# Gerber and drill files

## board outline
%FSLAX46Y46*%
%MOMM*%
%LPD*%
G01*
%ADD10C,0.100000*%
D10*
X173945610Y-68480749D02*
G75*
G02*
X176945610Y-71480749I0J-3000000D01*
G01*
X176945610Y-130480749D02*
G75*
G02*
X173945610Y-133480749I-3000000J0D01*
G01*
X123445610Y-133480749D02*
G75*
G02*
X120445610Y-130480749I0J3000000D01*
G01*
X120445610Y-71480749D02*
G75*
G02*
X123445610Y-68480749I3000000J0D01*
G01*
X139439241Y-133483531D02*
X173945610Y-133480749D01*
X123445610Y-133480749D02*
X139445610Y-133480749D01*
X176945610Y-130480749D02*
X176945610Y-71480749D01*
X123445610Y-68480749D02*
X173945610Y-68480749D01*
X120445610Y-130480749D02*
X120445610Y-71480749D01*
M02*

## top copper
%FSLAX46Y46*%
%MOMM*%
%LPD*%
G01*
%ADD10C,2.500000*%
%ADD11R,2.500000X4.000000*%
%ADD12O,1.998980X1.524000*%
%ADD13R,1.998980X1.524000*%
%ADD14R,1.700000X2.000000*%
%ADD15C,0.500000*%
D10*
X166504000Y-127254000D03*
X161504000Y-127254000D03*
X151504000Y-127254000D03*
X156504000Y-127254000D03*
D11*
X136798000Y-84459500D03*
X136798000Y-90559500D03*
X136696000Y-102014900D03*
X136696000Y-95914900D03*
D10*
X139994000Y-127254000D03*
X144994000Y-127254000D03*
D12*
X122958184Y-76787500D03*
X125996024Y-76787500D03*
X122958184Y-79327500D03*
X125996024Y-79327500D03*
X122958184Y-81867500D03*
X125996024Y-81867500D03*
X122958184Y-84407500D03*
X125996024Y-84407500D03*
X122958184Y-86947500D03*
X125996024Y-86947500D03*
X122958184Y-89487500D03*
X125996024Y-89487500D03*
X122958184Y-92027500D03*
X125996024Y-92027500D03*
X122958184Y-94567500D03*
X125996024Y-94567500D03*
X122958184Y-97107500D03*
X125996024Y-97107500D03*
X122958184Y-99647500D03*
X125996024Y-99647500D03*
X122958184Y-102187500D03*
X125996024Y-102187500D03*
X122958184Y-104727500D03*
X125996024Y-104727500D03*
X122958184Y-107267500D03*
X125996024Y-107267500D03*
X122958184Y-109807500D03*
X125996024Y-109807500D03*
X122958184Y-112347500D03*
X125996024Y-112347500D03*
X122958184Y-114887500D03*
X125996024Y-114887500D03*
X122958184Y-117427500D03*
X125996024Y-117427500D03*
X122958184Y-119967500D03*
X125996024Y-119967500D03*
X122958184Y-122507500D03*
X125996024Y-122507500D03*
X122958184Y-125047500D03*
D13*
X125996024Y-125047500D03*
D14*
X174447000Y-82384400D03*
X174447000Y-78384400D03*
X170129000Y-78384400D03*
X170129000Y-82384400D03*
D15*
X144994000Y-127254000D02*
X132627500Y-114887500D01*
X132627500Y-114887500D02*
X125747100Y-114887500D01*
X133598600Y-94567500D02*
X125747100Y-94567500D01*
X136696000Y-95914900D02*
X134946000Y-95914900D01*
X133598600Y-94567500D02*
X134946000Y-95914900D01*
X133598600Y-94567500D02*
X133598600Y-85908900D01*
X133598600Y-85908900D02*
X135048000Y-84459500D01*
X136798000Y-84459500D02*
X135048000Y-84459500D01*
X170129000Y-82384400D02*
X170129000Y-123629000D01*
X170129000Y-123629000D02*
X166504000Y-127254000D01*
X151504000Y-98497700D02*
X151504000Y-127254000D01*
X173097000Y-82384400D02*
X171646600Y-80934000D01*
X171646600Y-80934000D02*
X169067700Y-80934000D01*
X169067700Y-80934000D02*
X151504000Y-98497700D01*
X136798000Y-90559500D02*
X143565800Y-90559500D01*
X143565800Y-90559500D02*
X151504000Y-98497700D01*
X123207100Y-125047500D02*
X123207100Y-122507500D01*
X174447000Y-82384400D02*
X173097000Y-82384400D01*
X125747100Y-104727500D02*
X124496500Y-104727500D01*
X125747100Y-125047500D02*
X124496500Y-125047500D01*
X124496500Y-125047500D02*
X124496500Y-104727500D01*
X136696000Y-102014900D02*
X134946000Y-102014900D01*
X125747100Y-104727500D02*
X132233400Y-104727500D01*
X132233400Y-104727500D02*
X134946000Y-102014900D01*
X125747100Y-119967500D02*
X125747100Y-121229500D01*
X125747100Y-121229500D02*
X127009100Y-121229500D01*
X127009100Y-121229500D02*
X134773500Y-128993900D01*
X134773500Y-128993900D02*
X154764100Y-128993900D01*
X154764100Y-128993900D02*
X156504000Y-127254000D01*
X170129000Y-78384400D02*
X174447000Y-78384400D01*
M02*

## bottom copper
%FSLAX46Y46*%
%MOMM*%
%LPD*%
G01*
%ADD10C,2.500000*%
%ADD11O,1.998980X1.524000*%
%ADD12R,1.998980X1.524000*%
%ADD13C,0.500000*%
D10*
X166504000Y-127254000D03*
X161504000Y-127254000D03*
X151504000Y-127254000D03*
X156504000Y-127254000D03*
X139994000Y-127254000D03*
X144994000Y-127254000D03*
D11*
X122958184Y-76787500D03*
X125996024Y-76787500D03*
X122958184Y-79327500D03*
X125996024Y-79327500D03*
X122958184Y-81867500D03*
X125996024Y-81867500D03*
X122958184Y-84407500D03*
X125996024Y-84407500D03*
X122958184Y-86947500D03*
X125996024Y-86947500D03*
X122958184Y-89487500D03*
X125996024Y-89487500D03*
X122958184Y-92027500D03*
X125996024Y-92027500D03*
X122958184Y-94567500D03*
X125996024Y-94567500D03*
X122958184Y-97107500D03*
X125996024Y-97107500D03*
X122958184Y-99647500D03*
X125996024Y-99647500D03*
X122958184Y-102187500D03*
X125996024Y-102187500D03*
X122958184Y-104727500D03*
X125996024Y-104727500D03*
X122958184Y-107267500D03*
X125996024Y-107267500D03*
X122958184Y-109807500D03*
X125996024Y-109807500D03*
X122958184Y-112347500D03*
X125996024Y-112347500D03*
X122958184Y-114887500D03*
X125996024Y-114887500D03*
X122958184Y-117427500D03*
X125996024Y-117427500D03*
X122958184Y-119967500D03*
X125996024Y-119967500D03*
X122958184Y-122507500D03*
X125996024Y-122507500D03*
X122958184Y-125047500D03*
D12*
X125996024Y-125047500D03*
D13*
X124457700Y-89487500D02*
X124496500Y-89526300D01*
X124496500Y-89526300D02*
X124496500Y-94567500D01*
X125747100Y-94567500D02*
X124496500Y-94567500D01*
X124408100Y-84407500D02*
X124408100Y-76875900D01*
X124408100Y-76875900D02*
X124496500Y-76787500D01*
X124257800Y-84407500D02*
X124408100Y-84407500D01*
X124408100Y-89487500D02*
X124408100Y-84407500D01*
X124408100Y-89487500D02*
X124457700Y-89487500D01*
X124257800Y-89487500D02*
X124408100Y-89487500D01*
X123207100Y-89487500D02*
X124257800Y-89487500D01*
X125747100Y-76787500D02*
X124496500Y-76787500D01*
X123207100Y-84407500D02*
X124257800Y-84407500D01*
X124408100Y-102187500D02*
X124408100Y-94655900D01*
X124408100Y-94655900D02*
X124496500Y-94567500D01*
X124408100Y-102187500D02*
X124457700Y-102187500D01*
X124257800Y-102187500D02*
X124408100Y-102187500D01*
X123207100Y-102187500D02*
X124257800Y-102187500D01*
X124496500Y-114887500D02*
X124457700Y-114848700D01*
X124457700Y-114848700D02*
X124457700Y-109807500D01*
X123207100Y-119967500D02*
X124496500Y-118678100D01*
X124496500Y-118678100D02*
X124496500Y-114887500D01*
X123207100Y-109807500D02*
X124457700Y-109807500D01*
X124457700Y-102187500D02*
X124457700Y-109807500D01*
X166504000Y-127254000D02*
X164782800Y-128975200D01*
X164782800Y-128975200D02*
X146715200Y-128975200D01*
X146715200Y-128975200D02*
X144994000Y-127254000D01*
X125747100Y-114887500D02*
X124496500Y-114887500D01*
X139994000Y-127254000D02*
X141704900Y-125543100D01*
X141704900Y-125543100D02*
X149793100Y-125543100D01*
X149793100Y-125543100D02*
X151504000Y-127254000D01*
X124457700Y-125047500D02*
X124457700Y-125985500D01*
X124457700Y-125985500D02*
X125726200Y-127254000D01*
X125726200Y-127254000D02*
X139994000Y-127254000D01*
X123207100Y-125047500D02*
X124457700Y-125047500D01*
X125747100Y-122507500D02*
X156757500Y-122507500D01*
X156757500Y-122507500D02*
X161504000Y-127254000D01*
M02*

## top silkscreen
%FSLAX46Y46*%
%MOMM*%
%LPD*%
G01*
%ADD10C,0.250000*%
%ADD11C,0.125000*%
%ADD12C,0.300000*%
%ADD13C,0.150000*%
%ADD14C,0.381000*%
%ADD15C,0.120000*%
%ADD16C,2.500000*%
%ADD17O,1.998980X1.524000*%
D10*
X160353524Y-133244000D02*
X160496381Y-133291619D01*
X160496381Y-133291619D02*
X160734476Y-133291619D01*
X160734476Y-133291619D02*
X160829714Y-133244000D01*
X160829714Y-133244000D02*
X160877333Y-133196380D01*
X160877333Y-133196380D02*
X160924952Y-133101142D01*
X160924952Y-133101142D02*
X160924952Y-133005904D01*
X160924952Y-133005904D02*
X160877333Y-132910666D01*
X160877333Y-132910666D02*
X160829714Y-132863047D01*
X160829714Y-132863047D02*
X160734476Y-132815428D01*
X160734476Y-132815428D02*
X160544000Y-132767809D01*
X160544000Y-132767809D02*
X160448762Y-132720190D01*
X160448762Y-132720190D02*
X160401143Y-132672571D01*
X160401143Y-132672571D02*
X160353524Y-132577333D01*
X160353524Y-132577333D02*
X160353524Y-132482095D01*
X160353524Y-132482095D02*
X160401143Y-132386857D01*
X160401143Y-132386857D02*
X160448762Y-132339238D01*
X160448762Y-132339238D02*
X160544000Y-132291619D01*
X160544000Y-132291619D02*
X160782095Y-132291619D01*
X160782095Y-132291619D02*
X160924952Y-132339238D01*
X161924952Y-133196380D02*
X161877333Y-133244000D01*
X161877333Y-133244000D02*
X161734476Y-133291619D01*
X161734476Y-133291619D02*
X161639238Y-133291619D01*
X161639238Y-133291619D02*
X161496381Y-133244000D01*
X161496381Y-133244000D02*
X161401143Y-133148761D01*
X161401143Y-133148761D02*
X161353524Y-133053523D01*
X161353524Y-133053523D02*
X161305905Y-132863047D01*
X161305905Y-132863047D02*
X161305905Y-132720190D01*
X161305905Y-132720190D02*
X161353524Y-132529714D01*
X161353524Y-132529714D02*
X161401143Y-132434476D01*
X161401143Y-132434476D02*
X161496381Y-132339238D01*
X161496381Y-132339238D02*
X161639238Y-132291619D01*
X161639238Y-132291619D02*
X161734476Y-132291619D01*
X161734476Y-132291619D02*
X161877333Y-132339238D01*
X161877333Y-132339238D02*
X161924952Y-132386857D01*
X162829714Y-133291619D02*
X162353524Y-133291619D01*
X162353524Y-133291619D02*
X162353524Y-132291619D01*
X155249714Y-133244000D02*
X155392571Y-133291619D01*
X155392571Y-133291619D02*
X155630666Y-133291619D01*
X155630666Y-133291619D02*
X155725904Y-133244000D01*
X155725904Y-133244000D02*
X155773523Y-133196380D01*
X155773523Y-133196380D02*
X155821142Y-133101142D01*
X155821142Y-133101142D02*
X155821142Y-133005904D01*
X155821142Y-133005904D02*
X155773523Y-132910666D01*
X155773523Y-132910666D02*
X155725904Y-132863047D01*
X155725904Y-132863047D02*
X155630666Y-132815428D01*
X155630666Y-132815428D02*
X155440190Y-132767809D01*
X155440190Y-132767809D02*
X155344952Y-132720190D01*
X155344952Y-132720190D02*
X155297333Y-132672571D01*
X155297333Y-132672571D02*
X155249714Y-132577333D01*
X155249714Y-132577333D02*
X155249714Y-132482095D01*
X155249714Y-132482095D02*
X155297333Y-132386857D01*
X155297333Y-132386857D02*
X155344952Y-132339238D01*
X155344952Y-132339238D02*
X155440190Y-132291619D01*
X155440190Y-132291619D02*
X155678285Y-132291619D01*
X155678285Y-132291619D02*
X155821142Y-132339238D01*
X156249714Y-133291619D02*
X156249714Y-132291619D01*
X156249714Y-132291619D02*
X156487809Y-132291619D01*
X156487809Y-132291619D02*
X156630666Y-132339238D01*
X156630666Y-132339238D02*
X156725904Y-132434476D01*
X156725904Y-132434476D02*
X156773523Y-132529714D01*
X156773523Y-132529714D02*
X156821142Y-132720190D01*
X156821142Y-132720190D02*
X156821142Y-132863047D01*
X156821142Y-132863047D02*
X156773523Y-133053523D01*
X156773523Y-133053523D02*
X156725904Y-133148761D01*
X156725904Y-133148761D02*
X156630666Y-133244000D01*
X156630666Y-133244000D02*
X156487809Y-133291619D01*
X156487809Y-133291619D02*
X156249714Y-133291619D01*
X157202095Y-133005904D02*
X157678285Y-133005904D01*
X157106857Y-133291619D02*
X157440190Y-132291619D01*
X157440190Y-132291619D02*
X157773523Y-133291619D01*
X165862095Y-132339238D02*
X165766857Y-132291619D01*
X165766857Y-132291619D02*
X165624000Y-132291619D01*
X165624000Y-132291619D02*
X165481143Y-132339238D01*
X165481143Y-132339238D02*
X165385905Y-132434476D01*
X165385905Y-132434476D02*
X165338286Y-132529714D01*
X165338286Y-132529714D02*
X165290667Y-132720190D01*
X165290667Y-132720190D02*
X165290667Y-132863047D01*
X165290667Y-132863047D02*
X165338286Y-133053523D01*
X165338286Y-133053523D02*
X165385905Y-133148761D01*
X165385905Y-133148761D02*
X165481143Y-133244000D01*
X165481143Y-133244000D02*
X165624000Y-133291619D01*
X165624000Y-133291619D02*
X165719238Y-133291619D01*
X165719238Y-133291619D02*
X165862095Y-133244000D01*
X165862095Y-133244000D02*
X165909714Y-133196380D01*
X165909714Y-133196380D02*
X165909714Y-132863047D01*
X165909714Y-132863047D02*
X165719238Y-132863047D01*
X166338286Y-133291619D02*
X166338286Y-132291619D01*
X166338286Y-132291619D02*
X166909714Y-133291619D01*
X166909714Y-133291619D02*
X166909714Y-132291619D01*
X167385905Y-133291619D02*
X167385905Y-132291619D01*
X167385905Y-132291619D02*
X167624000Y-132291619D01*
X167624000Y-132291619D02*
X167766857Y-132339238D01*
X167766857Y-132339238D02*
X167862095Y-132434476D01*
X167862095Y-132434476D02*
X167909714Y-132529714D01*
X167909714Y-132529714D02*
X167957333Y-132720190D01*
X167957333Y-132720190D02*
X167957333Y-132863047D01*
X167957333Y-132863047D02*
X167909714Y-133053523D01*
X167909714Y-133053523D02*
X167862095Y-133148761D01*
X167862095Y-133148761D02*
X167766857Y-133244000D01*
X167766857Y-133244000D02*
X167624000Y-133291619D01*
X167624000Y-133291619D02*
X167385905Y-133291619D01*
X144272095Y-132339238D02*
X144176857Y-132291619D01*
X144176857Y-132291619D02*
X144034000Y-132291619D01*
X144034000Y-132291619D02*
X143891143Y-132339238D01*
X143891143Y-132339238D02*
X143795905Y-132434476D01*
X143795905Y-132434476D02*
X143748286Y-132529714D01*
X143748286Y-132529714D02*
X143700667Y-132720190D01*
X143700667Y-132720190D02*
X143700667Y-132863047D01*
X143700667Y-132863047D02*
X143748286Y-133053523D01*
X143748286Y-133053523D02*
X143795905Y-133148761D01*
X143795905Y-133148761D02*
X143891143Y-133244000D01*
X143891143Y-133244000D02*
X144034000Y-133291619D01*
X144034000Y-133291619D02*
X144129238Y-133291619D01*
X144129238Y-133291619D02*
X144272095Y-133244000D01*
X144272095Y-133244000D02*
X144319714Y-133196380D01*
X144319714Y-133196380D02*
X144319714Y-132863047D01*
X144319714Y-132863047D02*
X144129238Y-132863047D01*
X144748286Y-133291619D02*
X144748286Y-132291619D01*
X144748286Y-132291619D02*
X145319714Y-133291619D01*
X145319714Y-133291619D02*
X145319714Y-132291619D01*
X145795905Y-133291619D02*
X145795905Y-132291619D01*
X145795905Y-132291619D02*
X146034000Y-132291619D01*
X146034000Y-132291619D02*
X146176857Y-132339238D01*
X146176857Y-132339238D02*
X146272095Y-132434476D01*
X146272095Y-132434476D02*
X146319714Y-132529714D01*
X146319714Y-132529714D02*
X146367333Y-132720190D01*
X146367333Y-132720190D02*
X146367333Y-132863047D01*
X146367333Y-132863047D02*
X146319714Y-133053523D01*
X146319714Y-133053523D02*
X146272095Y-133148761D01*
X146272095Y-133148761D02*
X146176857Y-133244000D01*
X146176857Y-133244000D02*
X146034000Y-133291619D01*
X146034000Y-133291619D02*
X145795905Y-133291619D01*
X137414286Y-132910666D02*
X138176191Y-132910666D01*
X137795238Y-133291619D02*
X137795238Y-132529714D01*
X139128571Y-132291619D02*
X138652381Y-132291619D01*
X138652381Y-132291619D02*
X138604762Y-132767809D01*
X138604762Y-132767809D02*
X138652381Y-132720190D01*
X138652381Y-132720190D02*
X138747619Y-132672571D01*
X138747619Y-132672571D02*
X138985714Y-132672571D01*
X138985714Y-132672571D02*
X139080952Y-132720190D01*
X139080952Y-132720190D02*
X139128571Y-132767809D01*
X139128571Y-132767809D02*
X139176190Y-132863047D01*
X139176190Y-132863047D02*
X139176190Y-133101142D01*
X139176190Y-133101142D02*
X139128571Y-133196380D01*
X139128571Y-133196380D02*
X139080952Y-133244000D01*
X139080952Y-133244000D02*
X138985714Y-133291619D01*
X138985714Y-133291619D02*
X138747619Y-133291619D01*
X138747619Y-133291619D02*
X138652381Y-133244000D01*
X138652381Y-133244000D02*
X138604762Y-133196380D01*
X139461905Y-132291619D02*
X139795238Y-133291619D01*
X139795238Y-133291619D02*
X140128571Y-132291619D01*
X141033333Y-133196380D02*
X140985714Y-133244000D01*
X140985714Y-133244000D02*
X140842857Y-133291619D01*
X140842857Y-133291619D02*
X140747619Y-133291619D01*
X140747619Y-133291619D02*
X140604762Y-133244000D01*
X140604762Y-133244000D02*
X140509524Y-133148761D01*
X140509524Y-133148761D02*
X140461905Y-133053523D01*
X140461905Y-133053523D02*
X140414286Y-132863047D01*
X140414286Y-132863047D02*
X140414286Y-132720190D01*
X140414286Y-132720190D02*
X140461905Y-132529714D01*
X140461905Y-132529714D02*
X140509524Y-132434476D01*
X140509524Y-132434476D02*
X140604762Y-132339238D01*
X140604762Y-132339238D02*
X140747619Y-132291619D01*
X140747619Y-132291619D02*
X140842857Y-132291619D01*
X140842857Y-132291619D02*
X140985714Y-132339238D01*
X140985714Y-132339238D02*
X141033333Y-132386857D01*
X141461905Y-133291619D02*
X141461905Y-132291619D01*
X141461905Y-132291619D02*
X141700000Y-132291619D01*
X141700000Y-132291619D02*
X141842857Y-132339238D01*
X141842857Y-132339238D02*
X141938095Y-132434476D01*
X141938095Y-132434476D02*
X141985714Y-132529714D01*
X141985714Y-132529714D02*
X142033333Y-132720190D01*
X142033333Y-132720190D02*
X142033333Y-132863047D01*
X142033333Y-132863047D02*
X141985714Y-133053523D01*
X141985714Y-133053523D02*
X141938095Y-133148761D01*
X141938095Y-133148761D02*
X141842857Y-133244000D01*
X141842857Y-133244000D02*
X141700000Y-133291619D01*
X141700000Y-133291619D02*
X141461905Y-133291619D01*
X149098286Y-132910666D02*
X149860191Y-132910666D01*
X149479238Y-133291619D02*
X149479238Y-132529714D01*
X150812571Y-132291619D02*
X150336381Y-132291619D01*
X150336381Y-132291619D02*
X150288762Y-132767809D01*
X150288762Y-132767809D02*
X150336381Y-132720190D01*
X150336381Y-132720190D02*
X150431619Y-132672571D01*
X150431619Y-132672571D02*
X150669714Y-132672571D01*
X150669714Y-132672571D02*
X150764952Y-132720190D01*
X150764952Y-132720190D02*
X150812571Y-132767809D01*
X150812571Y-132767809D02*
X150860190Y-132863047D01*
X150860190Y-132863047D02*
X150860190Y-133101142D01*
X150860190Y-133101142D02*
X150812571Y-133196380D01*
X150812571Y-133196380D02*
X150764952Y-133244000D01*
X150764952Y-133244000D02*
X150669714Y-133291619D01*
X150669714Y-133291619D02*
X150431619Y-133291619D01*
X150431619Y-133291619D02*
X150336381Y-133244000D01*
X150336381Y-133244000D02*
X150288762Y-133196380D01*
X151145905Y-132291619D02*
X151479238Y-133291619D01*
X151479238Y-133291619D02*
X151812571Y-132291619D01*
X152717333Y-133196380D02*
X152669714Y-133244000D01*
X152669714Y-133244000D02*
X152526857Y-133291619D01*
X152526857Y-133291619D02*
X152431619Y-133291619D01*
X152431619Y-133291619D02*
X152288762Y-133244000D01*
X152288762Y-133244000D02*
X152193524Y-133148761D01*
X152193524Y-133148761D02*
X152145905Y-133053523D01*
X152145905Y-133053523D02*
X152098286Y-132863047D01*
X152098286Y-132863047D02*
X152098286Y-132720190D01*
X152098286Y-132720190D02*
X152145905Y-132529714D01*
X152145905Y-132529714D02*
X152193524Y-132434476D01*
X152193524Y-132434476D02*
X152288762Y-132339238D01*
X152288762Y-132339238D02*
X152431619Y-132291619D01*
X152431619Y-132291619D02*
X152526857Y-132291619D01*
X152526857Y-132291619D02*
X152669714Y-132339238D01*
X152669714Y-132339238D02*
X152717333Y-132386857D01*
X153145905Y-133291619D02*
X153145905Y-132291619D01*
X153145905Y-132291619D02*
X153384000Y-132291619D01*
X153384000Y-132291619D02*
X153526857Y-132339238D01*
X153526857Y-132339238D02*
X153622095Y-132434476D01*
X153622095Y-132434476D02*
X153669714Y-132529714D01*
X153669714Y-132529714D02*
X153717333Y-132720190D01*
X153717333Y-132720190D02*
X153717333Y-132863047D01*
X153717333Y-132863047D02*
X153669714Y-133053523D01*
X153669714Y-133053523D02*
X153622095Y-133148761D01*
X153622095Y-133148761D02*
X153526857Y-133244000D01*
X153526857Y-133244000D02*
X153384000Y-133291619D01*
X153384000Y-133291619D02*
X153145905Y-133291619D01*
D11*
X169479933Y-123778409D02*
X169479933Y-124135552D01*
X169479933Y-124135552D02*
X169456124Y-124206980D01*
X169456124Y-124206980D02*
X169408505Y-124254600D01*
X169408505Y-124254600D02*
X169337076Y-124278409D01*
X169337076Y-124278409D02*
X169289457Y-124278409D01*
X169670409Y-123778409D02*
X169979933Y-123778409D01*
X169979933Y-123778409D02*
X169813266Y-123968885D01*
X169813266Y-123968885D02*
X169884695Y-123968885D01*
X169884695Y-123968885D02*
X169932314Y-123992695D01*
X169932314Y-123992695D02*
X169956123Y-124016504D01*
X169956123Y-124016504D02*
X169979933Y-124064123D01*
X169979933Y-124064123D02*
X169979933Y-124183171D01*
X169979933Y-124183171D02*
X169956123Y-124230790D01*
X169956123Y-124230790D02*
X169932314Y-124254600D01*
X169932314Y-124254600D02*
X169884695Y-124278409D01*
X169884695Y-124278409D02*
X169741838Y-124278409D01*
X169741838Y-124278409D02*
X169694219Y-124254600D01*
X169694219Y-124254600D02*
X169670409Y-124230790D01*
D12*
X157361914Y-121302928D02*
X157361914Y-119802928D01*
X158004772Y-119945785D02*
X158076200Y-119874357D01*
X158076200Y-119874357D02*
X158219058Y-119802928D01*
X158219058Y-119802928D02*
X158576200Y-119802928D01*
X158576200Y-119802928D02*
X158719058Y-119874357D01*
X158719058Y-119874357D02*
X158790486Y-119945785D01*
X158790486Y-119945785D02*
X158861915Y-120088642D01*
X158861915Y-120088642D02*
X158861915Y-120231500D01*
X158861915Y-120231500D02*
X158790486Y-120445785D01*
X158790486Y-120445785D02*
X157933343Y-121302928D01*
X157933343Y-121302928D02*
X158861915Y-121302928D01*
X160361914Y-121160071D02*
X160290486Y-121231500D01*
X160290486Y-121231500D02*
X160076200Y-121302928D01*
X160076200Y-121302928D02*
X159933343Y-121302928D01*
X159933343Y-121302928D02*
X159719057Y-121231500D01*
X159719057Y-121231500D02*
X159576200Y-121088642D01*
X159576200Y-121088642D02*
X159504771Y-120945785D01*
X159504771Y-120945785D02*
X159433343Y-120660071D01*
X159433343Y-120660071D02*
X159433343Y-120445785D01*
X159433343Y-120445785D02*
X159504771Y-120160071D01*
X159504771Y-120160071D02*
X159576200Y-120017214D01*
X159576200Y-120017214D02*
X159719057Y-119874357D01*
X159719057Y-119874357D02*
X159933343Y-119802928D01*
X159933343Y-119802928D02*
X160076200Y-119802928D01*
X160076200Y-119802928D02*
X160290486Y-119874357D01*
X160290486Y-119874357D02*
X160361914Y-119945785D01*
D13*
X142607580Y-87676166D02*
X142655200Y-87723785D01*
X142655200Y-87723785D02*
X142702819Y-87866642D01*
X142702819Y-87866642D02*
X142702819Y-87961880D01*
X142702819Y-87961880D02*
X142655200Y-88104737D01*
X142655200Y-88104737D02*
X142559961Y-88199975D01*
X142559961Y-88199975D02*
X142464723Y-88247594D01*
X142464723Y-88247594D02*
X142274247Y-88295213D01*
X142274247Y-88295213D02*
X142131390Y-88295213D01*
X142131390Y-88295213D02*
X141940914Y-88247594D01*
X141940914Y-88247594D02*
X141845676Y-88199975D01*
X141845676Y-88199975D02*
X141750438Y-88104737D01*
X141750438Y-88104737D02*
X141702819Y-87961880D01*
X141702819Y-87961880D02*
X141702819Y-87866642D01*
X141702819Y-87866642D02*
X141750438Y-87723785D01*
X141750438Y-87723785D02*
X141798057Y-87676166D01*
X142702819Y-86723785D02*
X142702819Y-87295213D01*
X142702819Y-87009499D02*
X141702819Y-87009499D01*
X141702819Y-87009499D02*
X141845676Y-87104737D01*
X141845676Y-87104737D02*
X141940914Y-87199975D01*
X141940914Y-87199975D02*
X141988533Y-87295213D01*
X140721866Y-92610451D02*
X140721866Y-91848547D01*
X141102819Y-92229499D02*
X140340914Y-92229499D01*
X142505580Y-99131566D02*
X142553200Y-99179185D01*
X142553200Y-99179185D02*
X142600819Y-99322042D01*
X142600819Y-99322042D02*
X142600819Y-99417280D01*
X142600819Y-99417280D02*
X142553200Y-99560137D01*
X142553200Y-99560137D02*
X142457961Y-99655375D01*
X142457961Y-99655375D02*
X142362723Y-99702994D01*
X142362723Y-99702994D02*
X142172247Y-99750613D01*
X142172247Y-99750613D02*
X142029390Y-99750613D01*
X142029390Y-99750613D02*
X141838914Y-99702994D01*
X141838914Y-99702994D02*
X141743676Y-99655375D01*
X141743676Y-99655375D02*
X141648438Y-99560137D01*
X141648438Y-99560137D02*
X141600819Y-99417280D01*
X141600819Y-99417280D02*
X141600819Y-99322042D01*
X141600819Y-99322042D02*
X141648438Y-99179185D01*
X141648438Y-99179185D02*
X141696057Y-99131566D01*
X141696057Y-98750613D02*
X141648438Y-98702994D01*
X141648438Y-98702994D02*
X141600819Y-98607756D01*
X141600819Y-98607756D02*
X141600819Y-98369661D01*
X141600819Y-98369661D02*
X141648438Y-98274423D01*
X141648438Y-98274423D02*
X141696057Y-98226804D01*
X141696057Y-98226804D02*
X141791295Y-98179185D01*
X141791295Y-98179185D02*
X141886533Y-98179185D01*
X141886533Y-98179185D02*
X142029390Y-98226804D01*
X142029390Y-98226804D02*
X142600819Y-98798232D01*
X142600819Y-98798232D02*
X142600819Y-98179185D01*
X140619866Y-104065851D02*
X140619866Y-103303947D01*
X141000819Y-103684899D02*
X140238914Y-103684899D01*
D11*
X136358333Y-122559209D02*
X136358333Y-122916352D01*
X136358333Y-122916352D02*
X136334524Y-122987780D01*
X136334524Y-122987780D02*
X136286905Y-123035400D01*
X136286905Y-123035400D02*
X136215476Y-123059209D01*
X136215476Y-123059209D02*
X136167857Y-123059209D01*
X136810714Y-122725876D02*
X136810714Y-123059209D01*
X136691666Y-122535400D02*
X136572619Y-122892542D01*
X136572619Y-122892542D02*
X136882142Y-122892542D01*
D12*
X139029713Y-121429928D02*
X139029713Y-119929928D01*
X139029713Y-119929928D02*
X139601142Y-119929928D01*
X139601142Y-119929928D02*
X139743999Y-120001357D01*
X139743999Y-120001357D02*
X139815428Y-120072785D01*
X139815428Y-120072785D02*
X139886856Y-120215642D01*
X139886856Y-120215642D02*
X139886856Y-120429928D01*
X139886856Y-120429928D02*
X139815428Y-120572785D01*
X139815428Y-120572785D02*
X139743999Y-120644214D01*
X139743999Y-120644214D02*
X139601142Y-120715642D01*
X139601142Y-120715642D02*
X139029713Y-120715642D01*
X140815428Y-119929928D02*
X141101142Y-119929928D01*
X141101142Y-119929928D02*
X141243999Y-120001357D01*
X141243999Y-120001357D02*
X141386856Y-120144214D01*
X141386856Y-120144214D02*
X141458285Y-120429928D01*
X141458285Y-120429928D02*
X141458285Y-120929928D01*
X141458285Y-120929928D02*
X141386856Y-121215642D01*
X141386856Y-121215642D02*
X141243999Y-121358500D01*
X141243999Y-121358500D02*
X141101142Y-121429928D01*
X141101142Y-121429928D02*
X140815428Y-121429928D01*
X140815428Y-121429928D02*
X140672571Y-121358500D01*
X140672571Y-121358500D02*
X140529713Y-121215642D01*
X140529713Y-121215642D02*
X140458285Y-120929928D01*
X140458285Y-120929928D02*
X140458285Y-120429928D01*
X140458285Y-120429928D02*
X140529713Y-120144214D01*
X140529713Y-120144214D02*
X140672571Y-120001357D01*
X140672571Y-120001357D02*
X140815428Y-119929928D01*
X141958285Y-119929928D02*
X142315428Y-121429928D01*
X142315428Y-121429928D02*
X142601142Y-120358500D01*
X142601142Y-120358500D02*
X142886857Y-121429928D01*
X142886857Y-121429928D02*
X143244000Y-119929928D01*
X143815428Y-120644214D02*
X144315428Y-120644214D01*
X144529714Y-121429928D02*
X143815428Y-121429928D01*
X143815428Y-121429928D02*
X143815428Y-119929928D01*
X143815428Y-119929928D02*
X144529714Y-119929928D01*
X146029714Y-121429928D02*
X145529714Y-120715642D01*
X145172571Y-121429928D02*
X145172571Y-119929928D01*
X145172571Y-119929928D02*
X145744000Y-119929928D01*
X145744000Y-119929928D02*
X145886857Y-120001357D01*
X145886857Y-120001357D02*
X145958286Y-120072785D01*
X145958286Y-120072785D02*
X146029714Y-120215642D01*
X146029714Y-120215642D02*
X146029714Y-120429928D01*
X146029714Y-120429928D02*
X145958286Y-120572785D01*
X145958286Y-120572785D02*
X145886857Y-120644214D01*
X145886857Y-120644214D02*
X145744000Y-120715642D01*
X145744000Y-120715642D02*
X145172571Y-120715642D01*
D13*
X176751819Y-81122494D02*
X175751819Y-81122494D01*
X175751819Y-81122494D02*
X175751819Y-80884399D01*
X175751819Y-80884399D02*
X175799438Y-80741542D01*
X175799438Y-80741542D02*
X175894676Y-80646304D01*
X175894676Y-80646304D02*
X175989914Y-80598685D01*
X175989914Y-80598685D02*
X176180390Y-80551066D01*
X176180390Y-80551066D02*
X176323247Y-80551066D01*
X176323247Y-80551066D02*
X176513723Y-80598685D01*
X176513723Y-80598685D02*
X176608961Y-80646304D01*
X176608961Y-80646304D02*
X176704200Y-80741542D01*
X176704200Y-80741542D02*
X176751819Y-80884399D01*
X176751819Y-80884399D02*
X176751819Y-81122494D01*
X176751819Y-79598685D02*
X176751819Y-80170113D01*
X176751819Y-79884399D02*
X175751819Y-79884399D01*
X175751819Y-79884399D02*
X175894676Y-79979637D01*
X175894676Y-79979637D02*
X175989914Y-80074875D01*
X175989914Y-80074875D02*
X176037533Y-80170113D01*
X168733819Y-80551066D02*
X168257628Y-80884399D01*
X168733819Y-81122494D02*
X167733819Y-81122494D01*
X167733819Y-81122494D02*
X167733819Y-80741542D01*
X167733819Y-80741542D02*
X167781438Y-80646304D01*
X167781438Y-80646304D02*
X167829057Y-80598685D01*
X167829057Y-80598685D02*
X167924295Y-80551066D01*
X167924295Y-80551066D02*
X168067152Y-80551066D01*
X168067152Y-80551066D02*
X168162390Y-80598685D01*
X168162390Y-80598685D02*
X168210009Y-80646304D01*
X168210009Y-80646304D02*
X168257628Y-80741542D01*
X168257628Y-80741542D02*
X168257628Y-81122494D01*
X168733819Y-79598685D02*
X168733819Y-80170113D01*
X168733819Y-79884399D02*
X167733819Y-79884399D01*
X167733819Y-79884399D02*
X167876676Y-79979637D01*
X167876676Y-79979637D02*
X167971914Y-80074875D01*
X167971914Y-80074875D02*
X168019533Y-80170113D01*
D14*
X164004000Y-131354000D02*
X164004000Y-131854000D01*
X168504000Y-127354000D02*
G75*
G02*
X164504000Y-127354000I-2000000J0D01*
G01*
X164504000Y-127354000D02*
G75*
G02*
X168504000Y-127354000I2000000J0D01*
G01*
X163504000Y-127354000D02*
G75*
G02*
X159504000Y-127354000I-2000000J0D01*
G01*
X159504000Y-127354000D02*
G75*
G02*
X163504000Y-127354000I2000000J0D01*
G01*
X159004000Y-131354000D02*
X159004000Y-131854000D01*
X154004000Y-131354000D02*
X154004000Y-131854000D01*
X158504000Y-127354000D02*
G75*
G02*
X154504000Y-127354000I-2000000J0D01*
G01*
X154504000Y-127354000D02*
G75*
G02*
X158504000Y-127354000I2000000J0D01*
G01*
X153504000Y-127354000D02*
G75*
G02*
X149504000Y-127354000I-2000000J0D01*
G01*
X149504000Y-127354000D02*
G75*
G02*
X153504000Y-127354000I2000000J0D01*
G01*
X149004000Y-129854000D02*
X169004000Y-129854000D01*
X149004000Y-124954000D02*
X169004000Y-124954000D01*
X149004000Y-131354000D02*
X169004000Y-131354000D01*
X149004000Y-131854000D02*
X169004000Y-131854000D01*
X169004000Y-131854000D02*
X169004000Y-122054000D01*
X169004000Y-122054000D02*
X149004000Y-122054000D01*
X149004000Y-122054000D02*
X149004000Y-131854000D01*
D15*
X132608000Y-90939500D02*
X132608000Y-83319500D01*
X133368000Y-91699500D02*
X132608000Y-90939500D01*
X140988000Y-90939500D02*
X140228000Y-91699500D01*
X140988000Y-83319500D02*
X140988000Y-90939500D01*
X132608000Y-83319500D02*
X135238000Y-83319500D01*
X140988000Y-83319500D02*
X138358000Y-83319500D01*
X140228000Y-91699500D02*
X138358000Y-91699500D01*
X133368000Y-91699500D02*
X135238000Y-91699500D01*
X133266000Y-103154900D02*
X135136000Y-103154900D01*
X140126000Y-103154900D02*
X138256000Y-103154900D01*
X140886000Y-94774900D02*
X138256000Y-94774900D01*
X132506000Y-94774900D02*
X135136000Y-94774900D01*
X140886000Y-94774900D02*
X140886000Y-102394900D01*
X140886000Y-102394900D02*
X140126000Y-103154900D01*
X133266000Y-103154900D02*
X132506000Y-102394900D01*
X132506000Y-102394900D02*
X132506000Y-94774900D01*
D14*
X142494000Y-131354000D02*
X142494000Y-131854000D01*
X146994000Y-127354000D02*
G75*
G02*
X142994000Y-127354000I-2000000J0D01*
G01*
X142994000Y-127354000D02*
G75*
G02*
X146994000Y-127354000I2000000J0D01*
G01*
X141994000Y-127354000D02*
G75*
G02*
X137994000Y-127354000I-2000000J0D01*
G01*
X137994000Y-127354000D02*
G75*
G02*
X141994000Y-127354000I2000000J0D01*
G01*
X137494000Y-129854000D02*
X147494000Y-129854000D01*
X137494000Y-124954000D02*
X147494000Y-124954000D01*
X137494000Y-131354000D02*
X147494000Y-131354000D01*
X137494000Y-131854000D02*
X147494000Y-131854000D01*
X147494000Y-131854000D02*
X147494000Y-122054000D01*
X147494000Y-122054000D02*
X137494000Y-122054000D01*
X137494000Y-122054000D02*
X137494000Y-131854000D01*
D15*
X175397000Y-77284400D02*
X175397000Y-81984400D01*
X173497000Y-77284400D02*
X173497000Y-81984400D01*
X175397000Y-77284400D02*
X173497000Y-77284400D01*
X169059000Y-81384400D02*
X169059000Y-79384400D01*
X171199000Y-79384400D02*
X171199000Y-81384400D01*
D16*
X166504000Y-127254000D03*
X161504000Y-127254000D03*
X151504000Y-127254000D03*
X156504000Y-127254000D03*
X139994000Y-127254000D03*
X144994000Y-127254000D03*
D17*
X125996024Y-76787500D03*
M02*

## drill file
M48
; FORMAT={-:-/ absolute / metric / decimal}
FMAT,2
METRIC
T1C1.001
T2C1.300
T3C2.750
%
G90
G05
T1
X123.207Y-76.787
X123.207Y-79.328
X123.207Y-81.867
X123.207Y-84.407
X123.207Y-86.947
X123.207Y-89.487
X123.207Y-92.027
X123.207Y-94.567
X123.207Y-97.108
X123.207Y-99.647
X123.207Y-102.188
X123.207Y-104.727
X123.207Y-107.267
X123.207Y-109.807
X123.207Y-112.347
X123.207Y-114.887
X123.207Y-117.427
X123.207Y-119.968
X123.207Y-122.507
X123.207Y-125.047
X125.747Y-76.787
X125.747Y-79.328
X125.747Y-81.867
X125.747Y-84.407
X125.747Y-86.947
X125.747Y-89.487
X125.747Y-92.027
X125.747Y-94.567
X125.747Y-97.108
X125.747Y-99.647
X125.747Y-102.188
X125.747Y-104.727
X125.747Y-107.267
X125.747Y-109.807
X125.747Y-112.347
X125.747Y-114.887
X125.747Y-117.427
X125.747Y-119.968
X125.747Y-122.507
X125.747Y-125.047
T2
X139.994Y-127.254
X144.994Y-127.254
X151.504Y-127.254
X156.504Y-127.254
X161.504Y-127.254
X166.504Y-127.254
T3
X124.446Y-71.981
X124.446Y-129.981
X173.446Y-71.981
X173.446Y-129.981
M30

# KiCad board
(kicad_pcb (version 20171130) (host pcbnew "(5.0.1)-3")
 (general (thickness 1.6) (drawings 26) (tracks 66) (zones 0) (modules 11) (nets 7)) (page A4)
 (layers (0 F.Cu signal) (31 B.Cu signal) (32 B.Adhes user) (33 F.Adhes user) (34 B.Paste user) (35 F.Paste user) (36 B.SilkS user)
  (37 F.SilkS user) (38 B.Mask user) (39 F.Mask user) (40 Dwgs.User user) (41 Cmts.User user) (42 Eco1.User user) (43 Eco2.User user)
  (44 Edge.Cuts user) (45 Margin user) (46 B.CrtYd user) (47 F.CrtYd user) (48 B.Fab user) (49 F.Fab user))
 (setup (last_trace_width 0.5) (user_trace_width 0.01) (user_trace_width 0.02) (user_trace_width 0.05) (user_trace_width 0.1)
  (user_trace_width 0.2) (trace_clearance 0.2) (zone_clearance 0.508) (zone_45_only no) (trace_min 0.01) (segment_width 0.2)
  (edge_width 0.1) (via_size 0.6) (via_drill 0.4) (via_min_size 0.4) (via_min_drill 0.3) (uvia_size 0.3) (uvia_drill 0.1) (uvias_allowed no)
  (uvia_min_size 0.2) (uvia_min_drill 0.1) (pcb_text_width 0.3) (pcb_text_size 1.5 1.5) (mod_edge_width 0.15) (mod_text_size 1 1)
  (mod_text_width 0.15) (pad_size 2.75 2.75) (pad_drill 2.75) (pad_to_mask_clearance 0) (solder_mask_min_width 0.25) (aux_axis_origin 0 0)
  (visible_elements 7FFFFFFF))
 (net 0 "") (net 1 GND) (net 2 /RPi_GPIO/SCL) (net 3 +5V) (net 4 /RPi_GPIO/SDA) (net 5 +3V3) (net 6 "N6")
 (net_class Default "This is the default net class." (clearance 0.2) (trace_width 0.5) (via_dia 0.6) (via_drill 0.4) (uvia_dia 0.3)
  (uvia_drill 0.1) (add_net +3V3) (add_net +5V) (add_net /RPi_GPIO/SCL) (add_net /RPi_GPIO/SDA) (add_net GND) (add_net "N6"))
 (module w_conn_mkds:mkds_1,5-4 (layer F.Cu) (at 159.004 127.254)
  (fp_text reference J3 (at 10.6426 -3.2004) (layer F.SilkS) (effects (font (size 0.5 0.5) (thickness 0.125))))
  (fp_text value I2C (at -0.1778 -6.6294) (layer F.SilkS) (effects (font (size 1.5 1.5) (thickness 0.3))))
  (fp_line (start 5 4.1) (end 5 4.6) (layer F.SilkS) (width 0.381))
  (fp_circle (center 7.5 0.1) (end 5.5 0.1) (layer F.SilkS) (width 0.381))
  (fp_circle (center 2.5 0.1) (end 0.5 0.1) (layer F.SilkS) (width 0.381))
  (fp_line (start 0 4.1) (end 0 4.6) (layer F.SilkS) (width 0.381))
  (fp_line (start -5 4.1) (end -5 4.6) (layer F.SilkS) (width 0.381))
  (fp_circle (center -2.5 0.1) (end -4.5 0.1) (layer F.SilkS) (width 0.381))
  (fp_circle (center -7.5 0.1) (end -5.5 0.1) (layer F.SilkS) (width 0.381))
  (fp_line (start -10 2.6) (end 10 2.6) (layer F.SilkS) (width 0.381))
  (fp_line (start -10 -2.3) (end 10 -2.3) (layer F.SilkS) (width 0.381))
  (fp_line (start -10 4.1) (end 10 4.1) (layer F.SilkS) (width 0.381))
  (fp_line (start -10 4.6) (end 10 4.6) (layer F.SilkS) (width 0.381))
  (fp_line (start 10 4.6) (end 10 -5.2) (layer F.SilkS) (width 0.381))
  (fp_line (start 10 -5.2) (end -10 -5.2) (layer F.SilkS) (width 0.381))
  (fp_line (start -10 -5.2) (end -10 4.6) (layer F.SilkS) (width 0.381))
  (pad 4 thru_hole circle (at 7.5 0) (size 2.5 2.5) (drill 1.3) (layers *.Cu *.Mask F.SilkS) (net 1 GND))
  (pad 3 thru_hole circle (at 2.5 0) (size 2.5 2.5) (drill 1.3) (layers *.Cu *.Mask F.SilkS) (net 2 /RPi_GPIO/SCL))
  (pad 1 thru_hole circle (at -7.5 0) (size 2.5 2.5) (drill 1.3) (layers *.Cu *.Mask F.SilkS) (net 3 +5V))
  (pad 2 thru_hole circle (at -2.5 0) (size 2.5 2.5) (drill 1.3) (layers *.Cu *.Mask F.SilkS) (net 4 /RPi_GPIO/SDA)))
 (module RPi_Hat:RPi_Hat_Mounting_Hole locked (layer F.Cu) (at 124.446 71.9807 90)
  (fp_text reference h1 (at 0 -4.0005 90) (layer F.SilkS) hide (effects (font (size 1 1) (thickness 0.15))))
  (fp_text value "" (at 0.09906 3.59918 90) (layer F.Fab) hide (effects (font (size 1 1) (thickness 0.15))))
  (pad "" np_thru_hole circle (at 0 0 90) (size 2.75 2.75) (drill 2.75) (layers *.Cu *.Mask) (solder_mask_margin 1.725) (clearance 1.725)))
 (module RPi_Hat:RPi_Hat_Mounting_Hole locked (layer F.Cu) (at 173.446 71.9807 90)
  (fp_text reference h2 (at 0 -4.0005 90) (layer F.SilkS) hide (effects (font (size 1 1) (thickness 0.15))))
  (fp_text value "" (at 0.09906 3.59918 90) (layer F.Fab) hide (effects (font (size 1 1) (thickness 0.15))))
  (pad "" np_thru_hole circle (at 0 0 90) (size 2.75 2.75) (drill 2.75) (layers *.Cu *.Mask) (solder_mask_margin 1.725) (clearance 1.725)))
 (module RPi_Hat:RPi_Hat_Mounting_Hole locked (layer F.Cu) (at 173.446 129.981 90)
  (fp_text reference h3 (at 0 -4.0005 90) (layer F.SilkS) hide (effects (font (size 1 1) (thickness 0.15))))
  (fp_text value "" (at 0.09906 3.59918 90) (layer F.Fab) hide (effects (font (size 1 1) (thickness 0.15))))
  (pad "" np_thru_hole circle (at 0 0 90) (size 2.75 2.75) (drill 2.75) (layers *.Cu *.Mask) (solder_mask_margin 1.725) (clearance 1.725)))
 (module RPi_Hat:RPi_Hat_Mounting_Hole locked (layer F.Cu) (at 124.446 129.981 90)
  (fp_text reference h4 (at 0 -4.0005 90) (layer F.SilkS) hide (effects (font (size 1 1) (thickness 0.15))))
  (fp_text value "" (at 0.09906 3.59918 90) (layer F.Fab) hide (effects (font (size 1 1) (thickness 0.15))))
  (pad "" np_thru_hole circle (at 0 0 90) (size 2.75 2.75) (drill 2.75) (layers *.Cu *.Mask) (solder_mask_margin 1.725) (clearance 1.725)))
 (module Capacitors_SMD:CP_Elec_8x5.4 (layer F.Cu) (at 136.798 87.5095 90)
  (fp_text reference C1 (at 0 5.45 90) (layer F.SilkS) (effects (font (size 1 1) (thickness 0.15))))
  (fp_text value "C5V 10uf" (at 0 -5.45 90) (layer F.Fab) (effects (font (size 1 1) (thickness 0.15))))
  (fp_line (start -3.43 -4.19) (end 4.19 -4.19) (layer F.SilkS) (width 0.12))
  (fp_line (start -4.19 -3.43) (end -3.43 -4.19) (layer F.SilkS) (width 0.12))
  (fp_line (start -3.43 4.19) (end -4.19 3.43) (layer F.SilkS) (width 0.12))
  (fp_line (start 4.19 4.19) (end -3.43 4.19) (layer F.SilkS) (width 0.12))
  (fp_line (start 4.19 -4.19) (end 4.19 -1.56) (layer F.SilkS) (width 0.12))
  (fp_line (start 4.19 4.19) (end 4.19 1.56) (layer F.SilkS) (width 0.12))
  (fp_line (start -4.19 3.43) (end -4.19 1.56) (layer F.SilkS) (width 0.12))
  (fp_line (start -4.19 -3.43) (end -4.19 -1.56) (layer F.SilkS) (width 0.12))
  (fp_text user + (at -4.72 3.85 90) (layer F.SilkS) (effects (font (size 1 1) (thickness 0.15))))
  (pad 2 smd rect (at 3.05 0 270) (size 4 2.5) (layers F.Cu F.Paste F.Mask) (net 1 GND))
  (pad 1 smd rect (at -3.05 0 270) (size 4 2.5) (layers F.Cu F.Paste F.Mask) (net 3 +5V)))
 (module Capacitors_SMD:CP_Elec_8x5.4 (layer F.Cu) (at 136.696 98.9649 90)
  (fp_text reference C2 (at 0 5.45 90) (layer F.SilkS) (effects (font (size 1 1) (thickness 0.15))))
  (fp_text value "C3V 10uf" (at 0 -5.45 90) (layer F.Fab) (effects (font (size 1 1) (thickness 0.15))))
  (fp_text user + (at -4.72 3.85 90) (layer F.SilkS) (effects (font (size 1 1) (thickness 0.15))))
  (fp_line (start -4.19 -3.43) (end -4.19 -1.56) (layer F.SilkS) (width 0.12))
  (fp_line (start -4.19 3.43) (end -4.19 1.56) (layer F.SilkS) (width 0.12))
  (fp_line (start 4.19 4.19) (end 4.19 1.56) (layer F.SilkS) (width 0.12))
  (fp_line (start 4.19 -4.19) (end 4.19 -1.56) (layer F.SilkS) (width 0.12))
  (fp_line (start 4.19 4.19) (end -3.43 4.19) (layer F.SilkS) (width 0.12))
  (fp_line (start -3.43 4.19) (end -4.19 3.43) (layer F.SilkS) (width 0.12))
  (fp_line (start -4.19 -3.43) (end -3.43 -4.19) (layer F.SilkS) (width 0.12))
  (fp_line (start -3.43 -4.19) (end 4.19 -4.19) (layer F.SilkS) (width 0.12))
  (pad 1 smd rect (at -3.05 0 270) (size 4 2.5) (layers F.Cu F.Paste F.Mask) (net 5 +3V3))
  (pad 2 smd rect (at 3.05 0 270) (size 4 2.5) (layers F.Cu F.Paste F.Mask) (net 1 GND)))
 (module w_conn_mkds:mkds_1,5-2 (layer F.Cu) (at 142.494 127.254)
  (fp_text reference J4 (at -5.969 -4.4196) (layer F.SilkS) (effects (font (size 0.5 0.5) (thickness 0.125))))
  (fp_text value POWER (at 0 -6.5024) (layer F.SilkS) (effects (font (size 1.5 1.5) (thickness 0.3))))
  (fp_line (start 0 4.1) (end 0 4.6) (layer F.SilkS) (width 0.381))
  (fp_circle (center 2.5 0.1) (end 0.5 0.1) (layer F.SilkS) (width 0.381))
  (fp_circle (center -2.5 0.1) (end -0.5 0.1) (layer F.SilkS) (width 0.381))
  (fp_line (start -5 2.6) (end 5 2.6) (layer F.SilkS) (width 0.381))
  (fp_line (start -5 -2.3) (end 5 -2.3) (layer F.SilkS) (width 0.381))
  (fp_line (start -5 4.1) (end 5 4.1) (layer F.SilkS) (width 0.381))
  (fp_line (start -5 4.6) (end 5 4.6) (layer F.SilkS) (width 0.381))
  (fp_line (start 5 4.6) (end 5 -5.2) (layer F.SilkS) (width 0.381))
  (fp_line (start 5 -5.2) (end -5 -5.2) (layer F.SilkS) (width 0.381))
  (fp_line (start -5 -5.2) (end -5 4.6) (layer F.SilkS) (width 0.381))
  (pad 1 thru_hole circle (at -2.5 0) (size 2.5 2.5) (drill 1.3) (layers *.Cu *.Mask F.SilkS) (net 3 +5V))
  (pad 2 thru_hole circle (at 2.5 0) (size 2.5 2.5) (drill 1.3) (layers *.Cu *.Mask F.SilkS) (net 1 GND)))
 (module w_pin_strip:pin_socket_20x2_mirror (layer B.Cu) (at 124.446 100.981 90)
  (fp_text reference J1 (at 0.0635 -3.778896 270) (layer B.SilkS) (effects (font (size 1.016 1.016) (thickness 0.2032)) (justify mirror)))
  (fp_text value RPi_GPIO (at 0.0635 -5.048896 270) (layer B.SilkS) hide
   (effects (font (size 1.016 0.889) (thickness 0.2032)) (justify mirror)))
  (pad 40 thru_hole oval (at 24.1935 -1.238896 270) (size 1.524 1.99898) (drill 1.00076 (offset 0 0.24892)) (layers *.Cu *.Mask B.SilkS))
  (pad 39 thru_hole oval (at 24.1935 1.301104 90) (size 1.524 1.99898) (drill 1.00076 (offset 0 0.24892)) (layers *.Cu *.Mask F.SilkS)
   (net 1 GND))
  (pad 38 thru_hole oval (at 21.6535 -1.238896 270) (size 1.524 1.99898) (drill 1.00076 (offset 0 0.24892)) (layers *.Cu *.Mask B.SilkS))
  (pad 37 thru_hole oval (at 21.6535 1.301104 270) (size 1.524 1.99898) (drill 1.00076 (offset 0 -0.24892)) (layers *.Cu *.Mask B.SilkS))
  (pad 36 thru_hole oval (at 19.1135 -1.238896 270) (size 1.524 1.99898) (drill 1.00076 (offset 0 0.24892)) (layers *.Cu *.Mask B.SilkS))
  (pad 35 thru_hole oval (at 19.1135 1.301104 270) (size 1.524 1.99898) (drill 1.00076 (offset 0 -0.24892)) (layers *.Cu *.Mask B.SilkS))
  (pad 34 thru_hole oval (at 16.5735 -1.238896 270) (size 1.524 1.99898) (drill 1.00076 (offset 0 0.24892)) (layers *.Cu *.Mask B.SilkS)
   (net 1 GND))
  (pad 33 thru_hole oval (at 16.5735 1.301104 270) (size 1.524 1.99898) (drill 1.00076 (offset 0 -0.24892)) (layers *.Cu *.Mask B.SilkS))
  (pad 32 thru_hole oval (at 14.0335 -1.238896 270) (size 1.524 1.99898) (drill 1.00076 (offset 0 0.24892)) (layers *.Cu *.Mask B.SilkS))
  (pad 31 thru_hole oval (at 14.0335 1.301104 270) (size 1.524 1.99898) (drill 1.00076 (offset 0 -0.24892)) (layers *.Cu *.Mask B.SilkS))
  (pad 30 thru_hole oval (at 11.4935 -1.238896 270) (size 1.524 1.99898) (drill 1.00076 (offset 0 0.24892)) (layers *.Cu *.Mask B.SilkS)
   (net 1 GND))
  (pad 29 thru_hole oval (at 11.4935 1.301104 270) (size 1.524 1.99898) (drill 1.00076 (offset 0 -0.24892)) (layers *.Cu *.Mask B.SilkS))
  (pad 28 thru_hole oval (at 8.9535 -1.238896 270) (size 1.524 1.99898) (drill 1.00076 (offset 0 0.24892)) (layers *.Cu *.Mask B.SilkS))
  (pad 27 thru_hole oval (at 8.9535 1.301104 270) (size 1.524 1.99898) (drill 1.00076 (offset 0 -0.24892)) (layers *.Cu *.Mask B.SilkS))
  (pad 26 thru_hole oval (at 6.4135 -1.238896 270) (size 1.524 1.99898) (drill 1.00076 (offset 0 0.24892)) (layers *.Cu *.Mask B.SilkS))
  (pad 25 thru_hole oval (at 6.4135 1.301104 270) (size 1.524 1.99898) (drill 1.00076 (offset 0 -0.24892)) (layers *.Cu *.Mask B.SilkS)
   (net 1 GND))
  (pad 24 thru_hole oval (at 3.8735 -1.238896 270) (size 1.524 1.99898) (drill 1.00076 (offset 0 0.24892)) (layers *.Cu *.Mask B.SilkS))
  (pad 23 thru_hole oval (at 3.8735 1.301104 270) (size 1.524 1.99898) (drill 1.00076 (offset 0 -0.24892)) (layers *.Cu *.Mask B.SilkS))
  (pad 22 thru_hole oval (at 1.3335 -1.238896 270) (size 1.524 1.99898) (drill 1.00076 (offset 0 0.24892)) (layers *.Cu *.Mask B.SilkS))
  (pad 21 thru_hole oval (at 1.3335 1.301104 270) (size 1.524 1.99898) (drill 1.00076 (offset 0 -0.24892)) (layers *.Cu *.Mask B.SilkS))
  (pad 20 thru_hole oval (at -1.2065 -1.238896 270) (size 1.524 1.99898) (drill 1.00076 (offset 0 0.24892)) (layers *.Cu *.Mask B.SilkS)
   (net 1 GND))
  (pad 19 thru_hole oval (at -1.2065 1.301104 270) (size 1.524 1.99898) (drill 1.00076 (offset 0 -0.24892)) (layers *.Cu *.Mask B.SilkS))
  (pad 18 thru_hole oval (at -3.7465 -1.238896 270) (size 1.524 1.99898) (drill 1.00076 (offset 0 0.24892)) (layers *.Cu *.Mask B.SilkS))
  (pad 17 thru_hole oval (at -3.7465 1.301104 270) (size 1.524 1.99898) (drill 1.00076 (offset 0 -0.24892)) (layers *.Cu *.Mask B.SilkS)
   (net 5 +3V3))
  (pad 16 thru_hole oval (at -6.2865 -1.238896 270) (size 1.524 1.99898) (drill 1.00076 (offset 0 0.24892)) (layers *.Cu *.Mask B.SilkS))
  (pad 15 thru_hole oval (at -6.2865 1.301104 270) (size 1.524 1.99898) (drill 1.00076 (offset 0 -0.24892)) (layers *.Cu *.Mask B.SilkS))
  (pad 14 thru_hole oval (at -8.8265 -1.238896 270) (size 1.524 1.99898) (drill 1.00076 (offset 0 0.24892)) (layers *.Cu *.Mask B.SilkS)
   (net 1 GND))
  (pad 13 thru_hole oval (at -8.8265 1.301104 270) (size 1.524 1.99898) (drill 1.00076 (offset 0 -0.24892)) (layers *.Cu *.Mask B.SilkS))
  (pad 12 thru_hole oval (at -11.3665 -1.238896 270) (size 1.524 1.99898) (drill 1.00076 (offset 0 0.24892)) (layers *.Cu *.Mask B.SilkS))
  (pad 11 thru_hole oval (at -11.3665 1.301104 270) (size 1.524 1.99898) (drill 1.00076 (offset 0 -0.24892)) (layers *.Cu *.Mask B.SilkS))
  (pad 10 thru_hole oval (at -13.9065 -1.238896 270) (size 1.524 1.99898) (drill 1.00076 (offset 0 0.24892)) (layers *.Cu *.Mask B.SilkS))
  (pad 9 thru_hole oval (at -13.9065 1.301104 270) (size 1.524 1.99898) (drill 1.00076 (offset 0 -0.24892)) (layers *.Cu *.Mask B.SilkS)
   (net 1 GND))
  (pad 8 thru_hole oval (at -16.4465 -1.238896 270) (size 1.524 1.99898) (drill 1.00076 (offset 0 0.24892)) (layers *.Cu *.Mask B.SilkS))
  (pad 7 thru_hole oval (at -16.4465 1.301104 270) (size 1.524 1.99898) (drill 1.00076 (offset 0 -0.24892)) (layers *.Cu *.Mask B.SilkS))
  (pad 6 thru_hole oval (at -18.9865 -1.238896 270) (size 1.524 1.99898) (drill 1.00076 (offset 0 0.24892)) (layers *.Cu *.Mask B.SilkS)
   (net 1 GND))
  (pad 5 thru_hole oval (at -18.9865 1.301104 270) (size 1.524 1.99898) (drill 1.00076 (offset 0 -0.24892)) (layers *.Cu *.Mask B.SilkS)
   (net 4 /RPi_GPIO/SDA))
  (pad 4 thru_hole oval (at -21.5265 -1.238896 270) (size 1.524 1.99898) (drill 1.00076 (offset 0 0.24892)) (layers *.Cu *.Mask B.SilkS)
   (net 3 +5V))
  (pad 3 thru_hole oval (at -21.5265 1.301104 270) (size 1.524 1.99898) (drill 1.00076 (offset 0 -0.24892)) (layers *.Cu *.Mask B.SilkS)
   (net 2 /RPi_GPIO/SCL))
  (pad 2 thru_hole oval (at -24.0665 -1.238896 270) (size 1.524 1.99898) (drill 1.00076 (offset 0 0.24892)) (layers *.Cu *.Mask B.SilkS)
   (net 3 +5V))
  (pad 1 thru_hole rect (at -24.0665 1.301104 270) (size 1.524 1.99898) (drill 1.00076 (offset 0 -0.24892)) (layers *.Cu *.Mask B.SilkS)
   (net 5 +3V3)))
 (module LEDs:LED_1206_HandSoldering (layer F.Cu) (at 174.447 80.3844 270)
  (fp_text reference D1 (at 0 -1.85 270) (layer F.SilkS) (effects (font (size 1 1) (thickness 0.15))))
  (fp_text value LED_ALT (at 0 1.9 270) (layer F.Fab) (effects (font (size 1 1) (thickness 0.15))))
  (fp_line (start -3.1 -0.95) (end 1.6 -0.95) (layer F.SilkS) (width 0.12))
  (fp_line (start -3.1 0.95) (end 1.6 0.95) (layer F.SilkS) (width 0.12))
  (fp_line (start -3.1 -0.95) (end -3.1 0.95) (layer F.SilkS) (width 0.12))
  (pad 2 smd rect (at 2 0 270) (size 2 1.7) (layers F.Cu F.Paste F.Mask) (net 3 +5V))
  (pad 1 smd rect (at -2 0 270) (size 2 1.7) (layers F.Cu F.Paste F.Mask) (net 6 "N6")))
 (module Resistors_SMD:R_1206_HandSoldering (layer F.Cu) (at 170.129 80.3844 90)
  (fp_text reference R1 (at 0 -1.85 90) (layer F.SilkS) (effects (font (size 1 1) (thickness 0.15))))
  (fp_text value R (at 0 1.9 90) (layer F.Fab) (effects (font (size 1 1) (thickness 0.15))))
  (fp_line (start -1 -1.07) (end 1 -1.07) (layer F.SilkS) (width 0.12))
  (fp_line (start 1 1.07) (end -1 1.07) (layer F.SilkS) (width 0.12))
  (pad 2 smd rect (at 2 0 90) (size 2 1.7) (layers F.Cu F.Paste F.Mask) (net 6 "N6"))
  (pad 1 smd rect (at -2 0 90) (size 2 1.7) (layers F.Cu F.Paste F.Mask) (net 1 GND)))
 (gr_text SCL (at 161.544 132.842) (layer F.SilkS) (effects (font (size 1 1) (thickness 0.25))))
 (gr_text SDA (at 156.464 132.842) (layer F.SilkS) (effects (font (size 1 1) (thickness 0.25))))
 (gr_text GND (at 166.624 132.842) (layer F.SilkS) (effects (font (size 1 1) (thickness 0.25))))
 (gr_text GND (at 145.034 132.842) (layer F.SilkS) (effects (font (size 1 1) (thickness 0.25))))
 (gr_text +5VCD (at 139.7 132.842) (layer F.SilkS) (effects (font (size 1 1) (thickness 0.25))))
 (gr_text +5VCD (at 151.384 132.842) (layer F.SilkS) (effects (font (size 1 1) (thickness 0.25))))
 (gr_arc (start 173.94561 71.480749) (end 173.94561 68.480749) (angle 90) (layer Edge.Cuts) (width 0.1))
 (gr_arc (start 173.94561 130.480749) (end 176.94561 130.480749) (angle 90) (layer Edge.Cuts) (width 0.1))
 (gr_arc (start 123.44561 130.480749) (end 123.44561 133.480749) (angle 90) (layer Edge.Cuts) (width 0.1))
 (gr_arc (start 123.44561 71.480749) (end 120.44561 71.480749) (angle 90) (layer Edge.Cuts) (width 0.1))
 (gr_line (start 139.439241 133.483531) (end 173.94561 133.480749) (layer Edge.Cuts) (width 0.1))
 (gr_line (start 123.44561 133.480749) (end 139.44561 133.480749) (layer Edge.Cuts) (width 0.1))
 (gr_line (start 176.94561 130.480749) (end 176.94561 71.480749) (angle 90) (layer Edge.Cuts) (width 0.1))
 (gr_line (start 123.44561 68.480749) (end 173.94561 68.480749) (angle 90) (layer Edge.Cuts) (width 0.1))
 (gr_line (start 120.44561 130.480749) (end 120.44561 71.480749) (angle 90) (layer Edge.Cuts) (width 0.1))
 (segment (start 124.4577 89.4875) (end 124.4965 89.5263) (width 0.5) (layer B.Cu) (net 1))
 (segment (start 124.4965 89.5263) (end 124.4965 94.5675) (width 0.5) (layer B.Cu) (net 1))
 (segment (start 125.7471 94.5675) (end 124.4965 94.5675) (width 0.5) (layer B.Cu) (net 1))
 (segment (start 124.4081 84.4075) (end 124.4081 76.8759) (width 0.5) (layer B.Cu) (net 1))
 (segment (start 124.4081 76.8759) (end 124.4965 76.7875) (width 0.5) (layer B.Cu) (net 1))
 (segment (start 124.2578 84.4075) (end 124.4081 84.4075) (width 0.5) (layer B.Cu) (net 1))
 (segment (start 124.4081 89.4875) (end 124.4081 84.4075) (width 0.5) (layer B.Cu) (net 1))
 (segment (start 124.4081 89.4875) (end 124.4577 89.4875) (width 0.5) (layer B.Cu) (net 1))
 (segment (start 124.2578 89.4875) (end 124.4081 89.4875) (width 0.5) (layer B.Cu) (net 1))
 (segment (start 123.2071 89.4875) (end 124.2578 89.4875) (width 0.5) (layer B.Cu) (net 1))
 (segment (start 125.7471 76.7875) (end 124.4965 76.7875) (width 0.5) (layer B.Cu) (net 1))
 (segment (start 123.2071 84.4075) (end 124.2578 84.4075) (width 0.5) (layer B.Cu) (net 1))
 (segment (start 144.994 127.254) (end 132.6275 114.8875) (width 0.5) (layer F.Cu) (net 1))
 (segment (start 132.6275 114.8875) (end 125.7471 114.8875) (width 0.5) (layer F.Cu) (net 1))
 (segment (start 124.4081 102.1875) (end 124.4081 94.6559) (width 0.5) (layer B.Cu) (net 1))
 (segment (start 124.4081 94.6559) (end 124.4965 94.5675) (width 0.5) (layer B.Cu) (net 1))
 (segment (start 124.4081 102.1875) (end 124.4577 102.1875) (width 0.5) (layer B.Cu) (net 1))
 (segment (start 124.2578 102.1875) (end 124.4081 102.1875) (width 0.5) (layer B.Cu) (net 1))
 (segment (start 123.2071 102.1875) (end 124.2578 102.1875) (width 0.5) (layer B.Cu) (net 1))
 (segment (start 133.5986 94.5675) (end 125.7471 94.5675) (width 0.5) (layer F.Cu) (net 1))
 (segment (start 124.4965 114.8875) (end 124.4577 114.8487) (width 0.5) (layer B.Cu) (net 1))
 (segment (start 124.4577 114.8487) (end 124.4577 109.8075) (width 0.5) (layer B.Cu) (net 1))
 (segment (start 123.2071 119.9675) (end 124.4965 118.6781) (width 0.5) (layer B.Cu) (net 1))
 (segment (start 124.4965 118.6781) (end 124.4965 114.8875) (width 0.5) (layer B.Cu) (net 1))
 (segment (start 123.2071 109.8075) (end 124.4577 109.8075) (width 0.5) (layer B.Cu) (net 1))
 (segment (start 124.4577 102.1875) (end 124.4577 109.8075) (width 0.5) (layer B.Cu) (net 1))
 (segment (start 166.504 127.254) (end 164.7828 128.9752) (width 0.5) (layer B.Cu) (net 1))
 (segment (start 164.7828 128.9752) (end 146.7152 128.9752) (width 0.5) (layer B.Cu) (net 1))
 (segment (start 146.7152 128.9752) (end 144.994 127.254) (width 0.5) (layer B.Cu) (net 1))
 (segment (start 136.696 95.9149) (end 134.946 95.9149) (width 0.5) (layer F.Cu) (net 1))
 (segment (start 133.5986 94.5675) (end 134.946 95.9149) (width 0.5) (layer F.Cu) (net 1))
 (segment (start 133.5986 94.5675) (end 133.5986 85.9089) (width 0.5) (layer F.Cu) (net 1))
 (segment (start 133.5986 85.9089) (end 135.048 84.4595) (width 0.5) (layer F.Cu) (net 1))
 (segment (start 125.7471 114.8875) (end 124.4965 114.8875) (width 0.5) (layer B.Cu) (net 1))
 (segment (start 136.798 84.4595) (end 135.048 84.4595) (width 0.5) (layer F.Cu) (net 1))
 (segment (start 170.129 82.3844) (end 170.129 123.629) (width 0.5) (layer F.Cu) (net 1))
 (segment (start 170.129 123.629) (end 166.504 127.254) (width 0.5) (layer F.Cu) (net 1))
 (segment (start 151.504 98.4977) (end 151.504 127.254) (width 0.5) (layer F.Cu) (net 3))
 (segment (start 173.097 82.3844) (end 171.6466 80.934) (width 0.5) (layer F.Cu) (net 3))
 (segment (start 171.6466 80.934) (end 169.0677 80.934) (width 0.5) (layer F.Cu) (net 3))
 (segment (start 169.0677 80.934) (end 151.504 98.4977) (width 0.5) (layer F.Cu) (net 3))
 (segment (start 136.798 90.5595) (end 143.5658 90.5595) (width 0.5) (layer F.Cu) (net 3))
 (segment (start 143.5658 90.5595) (end 151.504 98.4977) (width 0.5) (layer F.Cu) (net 3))
 (segment (start 139.994 127.254) (end 141.7049 125.5431) (width 0.5) (layer B.Cu) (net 3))
 (segment (start 141.7049 125.5431) (end 149.7931 125.5431) (width 0.5) (layer B.Cu) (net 3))
 (segment (start 149.7931 125.5431) (end 151.504 127.254) (width 0.5) (layer B.Cu) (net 3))
 (segment (start 124.4577 125.0475) (end 124.4577 125.9855) (width 0.5) (layer B.Cu) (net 3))
 (segment (start 124.4577 125.9855) (end 125.7262 127.254) (width 0.5) (layer B.Cu) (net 3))
 (segment (start 125.7262 127.254) (end 139.994 127.254) (width 0.5) (layer B.Cu) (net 3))
 (segment (start 123.2071 125.0475) (end 124.4577 125.0475) (width 0.5) (layer B.Cu) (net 3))
 (segment (start 123.2071 125.0475) (end 123.2071 122.5075) (width 0.5) (layer F.Cu) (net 3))
 (segment (start 174.447 82.3844) (end 173.097 82.3844) (width 0.5) (layer F.Cu) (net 3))
 (segment (start 125.7471 104.7275) (end 124.4965 104.7275) (width 0.5) (layer F.Cu) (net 5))
 (segment (start 125.7471 125.0475) (end 124.4965 125.0475) (width 0.5) (layer F.Cu) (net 5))
 (segment (start 124.4965 125.0475) (end 124.4965 104.7275) (width 0.5) (layer F.Cu) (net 5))
 (segment (start 136.696 102.0149) (end 134.946 102.0149) (width 0.5) (layer F.Cu) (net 5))
 (segment (start 125.7471 104.7275) (end 132.2334 104.7275) (width 0.5) (layer F.Cu) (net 5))
 (segment (start 132.2334 104.7275) (end 134.946 102.0149) (width 0.5) (layer F.Cu) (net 5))
 (segment (start 125.7471 122.5075) (end 156.7575 122.5075) (width 0.5) (layer B.Cu) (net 2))
 (segment (start 156.7575 122.5075) (end 161.504 127.254) (width 0.5) (layer B.Cu) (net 2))
 (segment (start 125.7471 119.9675) (end 125.7471 121.2295) (width 0.5) (layer F.Cu) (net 4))
 (segment (start 125.7471 121.2295) (end 127.0091 121.2295) (width 0.5) (layer F.Cu) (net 4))
 (segment (start 127.0091 121.2295) (end 134.7735 128.9939) (width 0.5) (layer F.Cu) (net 4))
 (segment (start 134.7735 128.9939) (end 154.7641 128.9939) (width 0.5) (layer F.Cu) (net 4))
 (segment (start 154.7641 128.9939) (end 156.504 127.254) (width 0.5) (layer F.Cu) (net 4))
 (segment (start 170.129 78.3844) (end 174.447 78.3844) (width 0.5) (layer F.Cu) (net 6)))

